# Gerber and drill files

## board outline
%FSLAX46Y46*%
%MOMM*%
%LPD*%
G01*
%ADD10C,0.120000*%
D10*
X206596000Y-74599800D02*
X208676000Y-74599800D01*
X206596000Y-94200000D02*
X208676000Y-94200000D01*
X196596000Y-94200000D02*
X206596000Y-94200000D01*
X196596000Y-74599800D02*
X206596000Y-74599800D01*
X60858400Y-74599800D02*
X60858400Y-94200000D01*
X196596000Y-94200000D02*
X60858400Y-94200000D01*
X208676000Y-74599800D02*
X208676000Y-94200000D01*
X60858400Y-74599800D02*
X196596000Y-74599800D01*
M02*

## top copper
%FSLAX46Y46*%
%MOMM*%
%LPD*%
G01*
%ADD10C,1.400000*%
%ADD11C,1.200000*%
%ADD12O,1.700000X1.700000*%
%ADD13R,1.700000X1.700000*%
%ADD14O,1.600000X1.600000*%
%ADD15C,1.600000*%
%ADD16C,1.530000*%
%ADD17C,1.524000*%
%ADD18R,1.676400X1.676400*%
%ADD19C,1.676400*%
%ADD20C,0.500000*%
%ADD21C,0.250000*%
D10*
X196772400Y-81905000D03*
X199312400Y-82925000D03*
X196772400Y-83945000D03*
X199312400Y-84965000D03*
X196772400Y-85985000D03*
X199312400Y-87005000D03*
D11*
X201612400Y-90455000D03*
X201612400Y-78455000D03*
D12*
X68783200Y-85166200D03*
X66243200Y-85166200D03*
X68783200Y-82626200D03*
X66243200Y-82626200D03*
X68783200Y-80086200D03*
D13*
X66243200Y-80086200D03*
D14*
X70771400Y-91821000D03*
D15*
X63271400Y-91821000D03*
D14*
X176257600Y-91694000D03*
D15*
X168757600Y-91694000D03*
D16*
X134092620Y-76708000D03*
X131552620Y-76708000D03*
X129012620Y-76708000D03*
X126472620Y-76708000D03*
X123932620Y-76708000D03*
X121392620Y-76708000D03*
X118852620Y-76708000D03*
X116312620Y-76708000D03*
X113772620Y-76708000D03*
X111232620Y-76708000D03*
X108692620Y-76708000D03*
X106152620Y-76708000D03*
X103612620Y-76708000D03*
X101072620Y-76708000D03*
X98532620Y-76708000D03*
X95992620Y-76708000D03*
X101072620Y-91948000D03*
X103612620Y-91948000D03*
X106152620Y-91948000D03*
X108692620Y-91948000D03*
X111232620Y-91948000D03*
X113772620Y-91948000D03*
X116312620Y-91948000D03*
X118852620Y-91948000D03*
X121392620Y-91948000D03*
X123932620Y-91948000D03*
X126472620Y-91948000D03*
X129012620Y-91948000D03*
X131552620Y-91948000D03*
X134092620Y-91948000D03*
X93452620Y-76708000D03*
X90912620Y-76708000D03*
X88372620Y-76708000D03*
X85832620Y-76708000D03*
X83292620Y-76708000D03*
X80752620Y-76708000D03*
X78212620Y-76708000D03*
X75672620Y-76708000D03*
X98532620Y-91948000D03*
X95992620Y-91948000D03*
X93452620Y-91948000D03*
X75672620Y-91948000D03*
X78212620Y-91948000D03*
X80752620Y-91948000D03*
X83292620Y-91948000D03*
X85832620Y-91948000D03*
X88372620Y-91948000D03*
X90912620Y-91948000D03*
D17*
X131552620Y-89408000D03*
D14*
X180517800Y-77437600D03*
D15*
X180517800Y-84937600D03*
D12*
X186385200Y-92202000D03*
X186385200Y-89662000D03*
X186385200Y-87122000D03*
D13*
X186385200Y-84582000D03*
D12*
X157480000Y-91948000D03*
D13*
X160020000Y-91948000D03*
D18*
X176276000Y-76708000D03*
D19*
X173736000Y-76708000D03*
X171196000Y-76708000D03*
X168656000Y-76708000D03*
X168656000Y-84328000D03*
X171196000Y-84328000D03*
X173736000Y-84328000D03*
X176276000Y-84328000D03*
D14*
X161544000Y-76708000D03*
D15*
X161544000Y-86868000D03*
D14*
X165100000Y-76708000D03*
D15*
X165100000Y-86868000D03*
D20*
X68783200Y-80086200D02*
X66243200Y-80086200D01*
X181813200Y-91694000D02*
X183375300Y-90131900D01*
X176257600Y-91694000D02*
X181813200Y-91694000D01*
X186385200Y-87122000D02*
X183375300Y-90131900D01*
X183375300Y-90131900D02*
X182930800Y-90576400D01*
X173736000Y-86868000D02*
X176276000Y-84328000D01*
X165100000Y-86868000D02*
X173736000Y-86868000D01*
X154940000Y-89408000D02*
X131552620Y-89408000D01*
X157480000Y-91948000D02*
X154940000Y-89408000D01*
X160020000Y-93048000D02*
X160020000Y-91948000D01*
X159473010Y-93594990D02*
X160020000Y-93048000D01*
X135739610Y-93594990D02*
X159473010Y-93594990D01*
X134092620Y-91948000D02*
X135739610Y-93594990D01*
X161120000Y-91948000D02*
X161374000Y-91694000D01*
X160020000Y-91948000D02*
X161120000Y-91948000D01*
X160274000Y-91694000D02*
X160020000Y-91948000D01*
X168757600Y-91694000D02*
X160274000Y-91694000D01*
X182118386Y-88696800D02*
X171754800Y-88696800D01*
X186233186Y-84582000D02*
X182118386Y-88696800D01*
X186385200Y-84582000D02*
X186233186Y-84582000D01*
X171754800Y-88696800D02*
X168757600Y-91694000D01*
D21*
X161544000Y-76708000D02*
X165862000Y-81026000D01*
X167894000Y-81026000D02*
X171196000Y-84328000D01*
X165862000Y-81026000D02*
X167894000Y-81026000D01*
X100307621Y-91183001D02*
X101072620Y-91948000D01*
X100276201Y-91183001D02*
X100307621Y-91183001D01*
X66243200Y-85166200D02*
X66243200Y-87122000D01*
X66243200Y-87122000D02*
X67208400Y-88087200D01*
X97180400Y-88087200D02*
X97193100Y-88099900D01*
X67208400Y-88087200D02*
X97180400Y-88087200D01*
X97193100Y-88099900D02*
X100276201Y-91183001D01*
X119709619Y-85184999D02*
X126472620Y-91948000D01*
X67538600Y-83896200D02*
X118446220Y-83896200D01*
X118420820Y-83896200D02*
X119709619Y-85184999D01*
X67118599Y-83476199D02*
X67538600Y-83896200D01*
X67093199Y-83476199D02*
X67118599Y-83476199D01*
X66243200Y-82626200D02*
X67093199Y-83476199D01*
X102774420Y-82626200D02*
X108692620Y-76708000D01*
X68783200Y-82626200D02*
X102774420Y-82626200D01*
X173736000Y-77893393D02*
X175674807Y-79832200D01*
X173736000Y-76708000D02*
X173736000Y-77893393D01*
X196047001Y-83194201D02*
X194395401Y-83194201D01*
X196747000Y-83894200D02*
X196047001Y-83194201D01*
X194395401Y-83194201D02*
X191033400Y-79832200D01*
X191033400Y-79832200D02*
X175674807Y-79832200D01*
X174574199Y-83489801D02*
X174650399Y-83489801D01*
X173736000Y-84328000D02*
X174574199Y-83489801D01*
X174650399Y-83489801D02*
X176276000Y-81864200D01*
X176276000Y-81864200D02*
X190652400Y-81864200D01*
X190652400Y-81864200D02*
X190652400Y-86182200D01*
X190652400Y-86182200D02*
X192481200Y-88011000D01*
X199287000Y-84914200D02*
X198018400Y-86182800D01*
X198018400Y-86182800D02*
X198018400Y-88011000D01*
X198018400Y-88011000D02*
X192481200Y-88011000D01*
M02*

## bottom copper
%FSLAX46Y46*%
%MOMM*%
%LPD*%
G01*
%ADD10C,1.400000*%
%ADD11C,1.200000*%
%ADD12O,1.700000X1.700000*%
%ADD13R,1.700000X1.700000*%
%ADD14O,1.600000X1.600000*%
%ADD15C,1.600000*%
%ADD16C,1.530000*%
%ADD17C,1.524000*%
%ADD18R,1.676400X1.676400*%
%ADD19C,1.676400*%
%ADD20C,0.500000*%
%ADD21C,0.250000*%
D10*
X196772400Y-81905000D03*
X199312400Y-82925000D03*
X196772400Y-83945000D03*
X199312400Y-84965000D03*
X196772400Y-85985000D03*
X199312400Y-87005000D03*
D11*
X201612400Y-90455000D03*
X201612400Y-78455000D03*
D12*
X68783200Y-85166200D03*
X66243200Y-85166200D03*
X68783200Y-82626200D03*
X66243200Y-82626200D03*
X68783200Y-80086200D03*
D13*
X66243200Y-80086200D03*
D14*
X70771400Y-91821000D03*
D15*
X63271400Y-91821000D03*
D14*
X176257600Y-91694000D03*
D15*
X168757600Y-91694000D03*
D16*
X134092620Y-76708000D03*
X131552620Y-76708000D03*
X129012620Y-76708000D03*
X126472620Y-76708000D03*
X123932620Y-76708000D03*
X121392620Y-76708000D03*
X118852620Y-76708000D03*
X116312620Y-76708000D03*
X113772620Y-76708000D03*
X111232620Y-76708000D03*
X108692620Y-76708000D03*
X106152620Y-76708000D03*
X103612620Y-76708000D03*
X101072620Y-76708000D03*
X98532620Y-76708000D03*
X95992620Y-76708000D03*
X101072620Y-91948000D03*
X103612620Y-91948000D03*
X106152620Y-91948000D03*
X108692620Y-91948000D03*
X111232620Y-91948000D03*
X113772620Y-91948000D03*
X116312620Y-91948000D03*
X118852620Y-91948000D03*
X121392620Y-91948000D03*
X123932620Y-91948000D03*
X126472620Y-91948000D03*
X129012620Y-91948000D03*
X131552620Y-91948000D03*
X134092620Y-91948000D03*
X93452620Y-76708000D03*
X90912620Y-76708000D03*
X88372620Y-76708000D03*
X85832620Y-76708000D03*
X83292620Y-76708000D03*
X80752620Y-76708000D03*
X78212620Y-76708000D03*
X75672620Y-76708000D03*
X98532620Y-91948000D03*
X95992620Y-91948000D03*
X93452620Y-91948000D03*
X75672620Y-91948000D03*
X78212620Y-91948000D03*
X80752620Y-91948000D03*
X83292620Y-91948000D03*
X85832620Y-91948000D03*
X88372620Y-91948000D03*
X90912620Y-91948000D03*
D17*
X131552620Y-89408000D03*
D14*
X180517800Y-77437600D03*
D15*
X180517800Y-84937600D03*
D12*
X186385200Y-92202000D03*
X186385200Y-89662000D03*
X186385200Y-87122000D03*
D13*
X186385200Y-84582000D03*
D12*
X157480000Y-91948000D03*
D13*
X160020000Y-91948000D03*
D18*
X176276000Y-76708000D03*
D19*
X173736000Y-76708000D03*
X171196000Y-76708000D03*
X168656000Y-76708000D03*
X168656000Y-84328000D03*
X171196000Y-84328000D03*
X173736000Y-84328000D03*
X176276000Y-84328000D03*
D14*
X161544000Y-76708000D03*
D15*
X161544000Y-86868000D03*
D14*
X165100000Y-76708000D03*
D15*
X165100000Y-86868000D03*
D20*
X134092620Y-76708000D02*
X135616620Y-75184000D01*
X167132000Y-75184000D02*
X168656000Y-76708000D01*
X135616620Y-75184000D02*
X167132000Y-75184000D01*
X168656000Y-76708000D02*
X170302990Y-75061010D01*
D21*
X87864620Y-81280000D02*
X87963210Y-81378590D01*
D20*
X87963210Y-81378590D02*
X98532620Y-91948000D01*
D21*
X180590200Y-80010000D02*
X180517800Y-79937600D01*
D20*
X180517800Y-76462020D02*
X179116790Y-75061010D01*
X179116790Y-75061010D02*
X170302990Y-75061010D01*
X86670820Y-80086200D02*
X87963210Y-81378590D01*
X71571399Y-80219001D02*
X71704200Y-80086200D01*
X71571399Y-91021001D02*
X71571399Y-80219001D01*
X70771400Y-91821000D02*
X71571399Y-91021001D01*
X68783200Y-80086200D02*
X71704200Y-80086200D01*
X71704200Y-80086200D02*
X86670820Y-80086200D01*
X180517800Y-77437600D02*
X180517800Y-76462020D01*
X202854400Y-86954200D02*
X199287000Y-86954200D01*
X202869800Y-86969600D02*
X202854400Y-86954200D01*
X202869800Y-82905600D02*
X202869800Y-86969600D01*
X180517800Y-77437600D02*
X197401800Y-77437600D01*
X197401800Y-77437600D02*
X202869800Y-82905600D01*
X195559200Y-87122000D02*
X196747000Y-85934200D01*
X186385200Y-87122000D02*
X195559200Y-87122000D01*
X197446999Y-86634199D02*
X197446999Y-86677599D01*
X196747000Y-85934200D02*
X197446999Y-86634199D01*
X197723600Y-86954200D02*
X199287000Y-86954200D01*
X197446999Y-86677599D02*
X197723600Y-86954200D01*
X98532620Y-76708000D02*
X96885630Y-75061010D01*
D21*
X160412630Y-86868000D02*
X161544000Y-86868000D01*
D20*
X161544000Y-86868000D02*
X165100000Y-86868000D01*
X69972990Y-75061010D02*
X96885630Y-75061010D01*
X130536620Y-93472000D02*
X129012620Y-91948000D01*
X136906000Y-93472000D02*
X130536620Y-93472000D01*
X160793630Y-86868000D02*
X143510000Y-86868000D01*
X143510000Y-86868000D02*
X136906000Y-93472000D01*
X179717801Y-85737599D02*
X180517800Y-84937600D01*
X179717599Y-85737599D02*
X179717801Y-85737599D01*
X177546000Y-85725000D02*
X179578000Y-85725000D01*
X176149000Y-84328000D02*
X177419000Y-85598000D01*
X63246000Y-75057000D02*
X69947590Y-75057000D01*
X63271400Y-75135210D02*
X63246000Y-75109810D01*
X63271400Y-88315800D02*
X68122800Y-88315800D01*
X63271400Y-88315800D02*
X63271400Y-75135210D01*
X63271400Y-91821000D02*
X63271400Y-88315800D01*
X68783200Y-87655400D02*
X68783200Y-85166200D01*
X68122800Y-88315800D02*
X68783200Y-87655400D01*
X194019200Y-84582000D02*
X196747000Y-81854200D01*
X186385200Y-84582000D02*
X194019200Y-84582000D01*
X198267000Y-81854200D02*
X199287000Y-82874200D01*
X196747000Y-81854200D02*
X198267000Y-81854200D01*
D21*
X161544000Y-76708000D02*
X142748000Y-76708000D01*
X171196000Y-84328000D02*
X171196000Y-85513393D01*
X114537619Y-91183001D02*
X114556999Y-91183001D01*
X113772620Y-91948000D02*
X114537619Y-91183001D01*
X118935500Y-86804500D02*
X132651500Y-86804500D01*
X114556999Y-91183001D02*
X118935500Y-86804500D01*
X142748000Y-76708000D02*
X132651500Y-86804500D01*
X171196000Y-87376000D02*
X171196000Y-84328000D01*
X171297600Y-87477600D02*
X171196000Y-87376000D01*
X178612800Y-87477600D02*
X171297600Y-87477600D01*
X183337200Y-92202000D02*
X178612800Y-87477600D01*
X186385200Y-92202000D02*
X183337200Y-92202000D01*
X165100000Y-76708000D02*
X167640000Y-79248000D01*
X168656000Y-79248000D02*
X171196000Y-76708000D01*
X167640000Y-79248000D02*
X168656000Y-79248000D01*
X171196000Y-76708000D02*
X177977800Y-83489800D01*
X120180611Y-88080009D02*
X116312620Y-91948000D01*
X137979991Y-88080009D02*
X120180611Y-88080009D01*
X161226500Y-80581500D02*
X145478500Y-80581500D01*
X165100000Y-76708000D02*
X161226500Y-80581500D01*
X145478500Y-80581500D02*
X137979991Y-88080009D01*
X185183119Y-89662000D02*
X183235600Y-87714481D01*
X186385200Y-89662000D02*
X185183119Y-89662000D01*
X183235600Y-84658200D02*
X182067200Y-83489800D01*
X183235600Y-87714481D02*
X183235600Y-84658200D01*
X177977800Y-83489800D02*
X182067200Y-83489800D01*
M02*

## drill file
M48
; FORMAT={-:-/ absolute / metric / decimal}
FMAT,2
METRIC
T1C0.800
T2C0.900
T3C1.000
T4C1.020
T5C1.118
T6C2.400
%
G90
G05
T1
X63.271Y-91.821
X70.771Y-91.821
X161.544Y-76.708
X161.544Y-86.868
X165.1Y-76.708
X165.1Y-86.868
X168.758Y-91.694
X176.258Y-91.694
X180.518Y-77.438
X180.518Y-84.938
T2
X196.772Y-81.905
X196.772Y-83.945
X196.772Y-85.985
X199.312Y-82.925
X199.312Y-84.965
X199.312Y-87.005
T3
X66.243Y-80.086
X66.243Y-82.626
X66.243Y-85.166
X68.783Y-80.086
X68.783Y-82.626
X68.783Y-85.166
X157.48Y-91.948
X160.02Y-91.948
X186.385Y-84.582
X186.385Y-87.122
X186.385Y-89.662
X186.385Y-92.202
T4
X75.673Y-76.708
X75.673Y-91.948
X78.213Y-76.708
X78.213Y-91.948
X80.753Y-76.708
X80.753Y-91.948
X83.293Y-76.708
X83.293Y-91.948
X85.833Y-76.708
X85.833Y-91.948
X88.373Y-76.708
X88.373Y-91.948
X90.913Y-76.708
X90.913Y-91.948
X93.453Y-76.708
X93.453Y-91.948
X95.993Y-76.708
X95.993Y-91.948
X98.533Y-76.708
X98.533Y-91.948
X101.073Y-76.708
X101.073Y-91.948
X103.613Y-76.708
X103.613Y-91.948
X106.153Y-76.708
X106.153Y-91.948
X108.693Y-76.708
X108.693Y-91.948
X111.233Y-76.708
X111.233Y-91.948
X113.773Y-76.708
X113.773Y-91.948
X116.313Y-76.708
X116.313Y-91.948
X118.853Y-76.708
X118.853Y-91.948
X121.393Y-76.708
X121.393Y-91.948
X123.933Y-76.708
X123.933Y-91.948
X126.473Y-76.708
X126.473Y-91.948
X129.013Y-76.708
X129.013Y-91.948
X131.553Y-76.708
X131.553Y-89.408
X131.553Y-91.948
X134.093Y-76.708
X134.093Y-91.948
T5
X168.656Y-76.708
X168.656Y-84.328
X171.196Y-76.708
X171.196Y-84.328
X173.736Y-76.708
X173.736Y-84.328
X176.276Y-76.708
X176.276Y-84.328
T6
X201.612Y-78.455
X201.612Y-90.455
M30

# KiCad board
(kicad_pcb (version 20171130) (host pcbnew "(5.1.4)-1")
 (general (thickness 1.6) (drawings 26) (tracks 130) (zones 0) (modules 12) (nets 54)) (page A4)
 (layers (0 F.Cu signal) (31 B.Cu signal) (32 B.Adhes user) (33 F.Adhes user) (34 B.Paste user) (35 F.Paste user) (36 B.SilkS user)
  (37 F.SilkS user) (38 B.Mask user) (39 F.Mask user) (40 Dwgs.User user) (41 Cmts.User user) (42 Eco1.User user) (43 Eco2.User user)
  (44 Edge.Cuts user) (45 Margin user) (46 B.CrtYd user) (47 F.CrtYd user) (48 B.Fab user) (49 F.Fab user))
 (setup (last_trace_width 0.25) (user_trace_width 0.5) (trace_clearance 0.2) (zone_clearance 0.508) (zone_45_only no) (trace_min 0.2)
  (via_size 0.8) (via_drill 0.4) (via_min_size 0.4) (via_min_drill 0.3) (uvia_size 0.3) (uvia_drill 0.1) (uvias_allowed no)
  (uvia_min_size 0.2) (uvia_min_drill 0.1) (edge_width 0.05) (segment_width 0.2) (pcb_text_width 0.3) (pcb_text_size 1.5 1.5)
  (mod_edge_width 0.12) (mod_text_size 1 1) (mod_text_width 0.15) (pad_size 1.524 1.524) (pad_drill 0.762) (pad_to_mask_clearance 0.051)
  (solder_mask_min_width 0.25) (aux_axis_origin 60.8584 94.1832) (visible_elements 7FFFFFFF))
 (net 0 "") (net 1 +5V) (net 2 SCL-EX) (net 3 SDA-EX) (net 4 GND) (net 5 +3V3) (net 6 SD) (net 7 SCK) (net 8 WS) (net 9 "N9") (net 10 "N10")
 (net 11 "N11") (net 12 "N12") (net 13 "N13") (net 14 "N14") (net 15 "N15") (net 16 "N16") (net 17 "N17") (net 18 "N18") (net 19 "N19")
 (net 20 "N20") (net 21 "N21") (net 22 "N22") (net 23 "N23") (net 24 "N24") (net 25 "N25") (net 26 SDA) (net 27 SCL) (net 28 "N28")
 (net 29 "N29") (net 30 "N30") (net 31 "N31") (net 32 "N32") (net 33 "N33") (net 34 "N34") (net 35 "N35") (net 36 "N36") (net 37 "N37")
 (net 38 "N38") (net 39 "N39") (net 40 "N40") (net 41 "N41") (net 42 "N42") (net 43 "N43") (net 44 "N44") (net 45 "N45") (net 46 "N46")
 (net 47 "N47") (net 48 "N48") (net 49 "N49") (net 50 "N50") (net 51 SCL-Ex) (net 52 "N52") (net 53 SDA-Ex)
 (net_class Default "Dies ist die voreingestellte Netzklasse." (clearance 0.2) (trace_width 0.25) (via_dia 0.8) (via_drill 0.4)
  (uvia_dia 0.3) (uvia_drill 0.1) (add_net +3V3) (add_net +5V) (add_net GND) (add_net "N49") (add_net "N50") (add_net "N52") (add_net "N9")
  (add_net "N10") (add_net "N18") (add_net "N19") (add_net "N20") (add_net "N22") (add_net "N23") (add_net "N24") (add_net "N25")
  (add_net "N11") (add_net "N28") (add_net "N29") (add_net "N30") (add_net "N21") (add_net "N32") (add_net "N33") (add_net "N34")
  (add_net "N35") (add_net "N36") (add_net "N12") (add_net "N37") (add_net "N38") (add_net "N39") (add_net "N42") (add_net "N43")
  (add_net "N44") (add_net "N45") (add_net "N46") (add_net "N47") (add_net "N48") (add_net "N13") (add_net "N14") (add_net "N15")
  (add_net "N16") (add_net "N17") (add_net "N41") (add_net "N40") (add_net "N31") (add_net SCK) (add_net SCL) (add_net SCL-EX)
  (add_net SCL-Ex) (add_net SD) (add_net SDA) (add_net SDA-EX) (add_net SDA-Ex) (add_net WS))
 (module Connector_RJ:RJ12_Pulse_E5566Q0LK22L (layer F.Cu) (at 200.8124 84.455 90)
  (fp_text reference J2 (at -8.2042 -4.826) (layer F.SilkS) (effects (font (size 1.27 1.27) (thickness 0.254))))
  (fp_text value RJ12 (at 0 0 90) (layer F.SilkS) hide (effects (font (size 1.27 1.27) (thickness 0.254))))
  (pad 1 thru_hole circle (at 2.55 -4.04 180) (size 1.4 1.4) (drill 0.9) (layers *.Cu *.Mask F.SilkS) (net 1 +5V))
  (pad 2 thru_hole circle (at 1.53 -1.5 180) (size 1.4 1.4) (drill 0.9) (layers *.Cu *.Mask F.SilkS) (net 1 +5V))
  (pad 3 thru_hole circle (at 0.51 -4.04 180) (size 1.4 1.4) (drill 0.9) (layers *.Cu *.Mask F.SilkS) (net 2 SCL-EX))
  (pad 4 thru_hole circle (at -0.51 -1.5 180) (size 1.4 1.4) (drill 0.9) (layers *.Cu *.Mask F.SilkS) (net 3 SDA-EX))
  (pad 5 thru_hole circle (at -1.53 -4.04 180) (size 1.4 1.4) (drill 0.9) (layers *.Cu *.Mask F.SilkS) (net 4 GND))
  (pad 6 thru_hole circle (at -2.55 -1.5 180) (size 1.4 1.4) (drill 0.9) (layers *.Cu *.Mask F.SilkS) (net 4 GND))
  (pad 7 thru_hole circle (at -6 0.8 180) (size 1.2 1.2) (drill 2.4) (layers *.Cu *.Mask F.SilkS))
  (pad 8 thru_hole circle (at 6 0.8 180) (size 1.2 1.2) (drill 2.4) (layers *.Cu *.Mask F.SilkS)))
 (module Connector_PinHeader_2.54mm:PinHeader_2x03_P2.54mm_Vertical (layer F.Cu) (at 66.2432 80.0862)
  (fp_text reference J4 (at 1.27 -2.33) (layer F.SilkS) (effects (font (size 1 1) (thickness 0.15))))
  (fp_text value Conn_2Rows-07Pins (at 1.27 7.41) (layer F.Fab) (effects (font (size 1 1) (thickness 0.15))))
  (pad 6 thru_hole oval (at 2.54 5.08) (size 1.7 1.7) (drill 1) (layers *.Cu *.Mask) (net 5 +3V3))
  (pad 5 thru_hole oval (at 0 5.08) (size 1.7 1.7) (drill 1) (layers *.Cu *.Mask) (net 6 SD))
  (pad 4 thru_hole oval (at 2.54 2.54) (size 1.7 1.7) (drill 1) (layers *.Cu *.Mask) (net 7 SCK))
  (pad 3 thru_hole oval (at 0 2.54) (size 1.7 1.7) (drill 1) (layers *.Cu *.Mask) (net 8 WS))
  (pad 2 thru_hole oval (at 2.54 0) (size 1.7 1.7) (drill 1) (layers *.Cu *.Mask) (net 4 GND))
  (pad 1 thru_hole rect (at 0 0) (size 1.7 1.7) (drill 1) (layers *.Cu *.Mask) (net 4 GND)))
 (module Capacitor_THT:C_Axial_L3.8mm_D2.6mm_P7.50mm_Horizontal (layer F.Cu) (at 63.2714 91.821)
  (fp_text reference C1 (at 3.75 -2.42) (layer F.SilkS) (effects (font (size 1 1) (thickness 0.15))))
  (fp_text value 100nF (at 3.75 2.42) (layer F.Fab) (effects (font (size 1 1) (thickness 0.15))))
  (pad 2 thru_hole oval (at 7.5 0) (size 1.6 1.6) (drill 0.8) (layers *.Cu *.Mask) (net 4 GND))
  (pad 1 thru_hole circle (at 0 0) (size 1.6 1.6) (drill 0.8) (layers *.Cu *.Mask) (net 5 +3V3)))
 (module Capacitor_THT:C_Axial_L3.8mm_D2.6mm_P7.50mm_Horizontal (layer F.Cu) (at 168.7576 91.694)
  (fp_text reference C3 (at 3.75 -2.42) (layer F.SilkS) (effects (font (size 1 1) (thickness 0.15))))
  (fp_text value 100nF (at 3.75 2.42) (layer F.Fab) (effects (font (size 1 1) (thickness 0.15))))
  (pad 2 thru_hole oval (at 7.5 0) (size 1.6 1.6) (drill 0.8) (layers *.Cu *.Mask) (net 4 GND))
  (pad 1 thru_hole circle (at 0 0) (size 1.6 1.6) (drill 0.8) (layers *.Cu *.Mask) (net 1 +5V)))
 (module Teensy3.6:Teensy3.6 (layer F.Cu) (at 104.88262 84.328 270)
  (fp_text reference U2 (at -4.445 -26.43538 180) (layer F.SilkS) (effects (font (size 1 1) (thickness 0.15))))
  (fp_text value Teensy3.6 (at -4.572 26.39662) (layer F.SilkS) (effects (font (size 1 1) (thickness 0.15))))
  (pad GND_1 thru_hole circle (at -7.62 -29.21 270) (size 1.53 1.53) (drill 1.02) (layers *.Cu *.Mask) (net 4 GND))
  (pad 0 thru_hole circle (at -7.62 -26.67 270) (size 1.53 1.53) (drill 1.02) (layers *.Cu *.Mask) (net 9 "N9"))
  (pad 1 thru_hole circle (at -7.62 -24.13 270) (size 1.53 1.53) (drill 1.02) (layers *.Cu *.Mask) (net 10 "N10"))
  (pad 2 thru_hole circle (at -7.62 -21.59 270) (size 1.53 1.53) (drill 1.02) (layers *.Cu *.Mask) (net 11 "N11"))
  (pad 3 thru_hole circle (at -7.62 -19.05 270) (size 1.53 1.53) (drill 1.02) (layers *.Cu *.Mask) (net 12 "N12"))
  (pad 4 thru_hole circle (at -7.62 -16.51 270) (size 1.53 1.53) (drill 1.02) (layers *.Cu *.Mask) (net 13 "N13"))
  (pad 5 thru_hole circle (at -7.62 -13.97 270) (size 1.53 1.53) (drill 1.02) (layers *.Cu *.Mask) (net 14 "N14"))
  (pad 6 thru_hole circle (at -7.62 -11.43 270) (size 1.53 1.53) (drill 1.02) (layers *.Cu *.Mask) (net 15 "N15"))
  (pad 7 thru_hole circle (at -7.62 -8.89 270) (size 1.53 1.53) (drill 1.02) (layers *.Cu *.Mask) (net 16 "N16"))
  (pad 8 thru_hole circle (at -7.62 -6.35 270) (size 1.53 1.53) (drill 1.02) (layers *.Cu *.Mask) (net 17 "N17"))
  (pad 9 thru_hole circle (at -7.62 -3.81 270) (size 1.53 1.53) (drill 1.02) (layers *.Cu *.Mask) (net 7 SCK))
  (pad 10 thru_hole circle (at -7.62 -1.27 270) (size 1.53 1.53) (drill 1.02) (layers *.Cu *.Mask) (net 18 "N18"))
  (pad 11 thru_hole circle (at -7.62 1.27 270) (size 1.53 1.53) (drill 1.02) (layers *.Cu *.Mask) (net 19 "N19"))
  (pad 12 thru_hole circle (at -7.62 3.81 270) (size 1.53 1.53) (drill 1.02) (layers *.Cu *.Mask) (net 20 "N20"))
  (pad 3V3_1 thru_hole circle (at -7.62 6.35 270) (size 1.53 1.53) (drill 1.02) (layers *.Cu *.Mask) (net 5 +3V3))
  (pad 24 thru_hole circle (at -7.62 8.89 270) (size 1.53 1.53) (drill 1.02) (layers *.Cu *.Mask) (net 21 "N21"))
  (pad 13 thru_hole circle (at 7.62 3.81 270) (size 1.53 1.53) (drill 1.02) (layers *.Cu *.Mask) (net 6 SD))
  (pad 14 thru_hole circle (at 7.62 1.27 270) (size 1.53 1.53) (drill 1.02) (layers *.Cu *.Mask) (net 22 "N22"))
  (pad 15 thru_hole circle (at 7.62 -1.27 270) (size 1.53 1.53) (drill 1.02) (layers *.Cu *.Mask) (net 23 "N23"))
  (pad 16 thru_hole circle (at 7.62 -3.81 270) (size 1.53 1.53) (drill 1.02) (layers *.Cu *.Mask) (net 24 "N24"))
  (pad 17 thru_hole circle (at 7.62 -6.35 270) (size 1.53 1.53) (drill 1.02) (layers *.Cu *.Mask) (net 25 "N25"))
  (pad 18 thru_hole circle (at 7.62 -8.89 270) (size 1.53 1.53) (drill 1.02) (layers *.Cu *.Mask) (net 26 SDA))
  (pad 19 thru_hole circle (at 7.62 -11.43 270) (size 1.53 1.53) (drill 1.02) (layers *.Cu *.Mask) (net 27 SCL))
  (pad 20 thru_hole circle (at 7.62 -13.97 270) (size 1.53 1.53) (drill 1.02) (layers *.Cu *.Mask) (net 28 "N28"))
  (pad 21 thru_hole circle (at 7.62 -16.51 270) (size 1.53 1.53) (drill 1.02) (layers *.Cu *.Mask) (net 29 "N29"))
  (pad 22 thru_hole circle (at 7.62 -19.05 270) (size 1.53 1.53) (drill 1.02) (layers *.Cu *.Mask) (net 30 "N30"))
  (pad 23 thru_hole circle (at 7.62 -21.59 270) (size 1.53 1.53) (drill 1.02) (layers *.Cu *.Mask) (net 8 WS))
  (pad 3V3_2 thru_hole circle (at 7.62 -24.13 270) (size 1.53 1.53) (drill 1.02) (layers *.Cu *.Mask) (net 5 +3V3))
  (pad AGND thru_hole circle (at 7.62 -26.67 270) (size 1.53 1.53) (drill 1.02) (layers *.Cu *.Mask) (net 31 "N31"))
  (pad VIN thru_hole circle (at 7.62 -29.21 270) (size 1.53 1.53) (drill 1.02) (layers *.Cu *.Mask) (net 1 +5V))
  (pad 25 thru_hole circle (at -7.62 11.43 270) (size 1.53 1.53) (drill 1.02) (layers *.Cu *.Mask) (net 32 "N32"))
  (pad 26 thru_hole circle (at -7.62 13.97 270) (size 1.53 1.53) (drill 1.02) (layers *.Cu *.Mask) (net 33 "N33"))
  (pad 27 thru_hole circle (at -7.62 16.51 270) (size 1.53 1.53) (drill 1.02) (layers *.Cu *.Mask) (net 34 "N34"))
  (pad 28 thru_hole circle (at -7.62 19.05 270) (size 1.53 1.53) (drill 1.02) (layers *.Cu *.Mask) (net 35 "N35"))
  (pad 29 thru_hole circle (at -7.62 21.59 270) (size 1.53 1.53) (drill 1.02) (layers *.Cu *.Mask) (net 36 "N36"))
  (pad 30 thru_hole circle (at -7.62 24.13 270) (size 1.53 1.53) (drill 1.02) (layers *.Cu *.Mask) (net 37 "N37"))
  (pad 31 thru_hole circle (at -7.62 26.67 270) (size 1.53 1.53) (drill 1.02) (layers *.Cu *.Mask) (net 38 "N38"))
  (pad 32 thru_hole circle (at -7.62 29.21 270) (size 1.53 1.53) (drill 1.02) (layers *.Cu *.Mask) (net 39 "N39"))
  (pad GND_2 thru_hole circle (at 7.62 6.35 270) (size 1.53 1.53) (drill 1.02) (layers *.Cu *.Mask) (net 4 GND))
  (pad A22 thru_hole circle (at 7.62 8.89 270) (size 1.53 1.53) (drill 1.02) (layers *.Cu *.Mask) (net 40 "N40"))
  (pad A21 thru_hole circle (at 7.62 11.43 270) (size 1.53 1.53) (drill 1.02) (layers *.Cu *.Mask) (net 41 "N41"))
  (pad 33 thru_hole circle (at 7.62 29.21 270) (size 1.53 1.53) (drill 1.02) (layers *.Cu *.Mask) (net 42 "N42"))
  (pad 34 thru_hole circle (at 7.62 26.67 270) (size 1.53 1.53) (drill 1.02) (layers *.Cu *.Mask) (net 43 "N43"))
  (pad 35 thru_hole circle (at 7.62 24.13 270) (size 1.53 1.53) (drill 1.02) (layers *.Cu *.Mask) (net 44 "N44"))
  (pad 36 thru_hole circle (at 7.62 21.59 270) (size 1.53 1.53) (drill 1.02) (layers *.Cu *.Mask) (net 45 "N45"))
  (pad 37 thru_hole circle (at 7.62 19.05 270) (size 1.53 1.53) (drill 1.02) (layers *.Cu *.Mask) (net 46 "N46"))
  (pad 38 thru_hole circle (at 7.62 16.51 270) (size 1.53 1.53) (drill 1.02) (layers *.Cu *.Mask) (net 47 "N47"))
  (pad 39 thru_hole circle (at 7.62 13.97 270) (size 1.53 1.53) (drill 1.02) (layers *.Cu *.Mask) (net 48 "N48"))
  (pad VUSB thru_hole circle (at 5.08 -26.67 270) (size 1.524 1.524) (drill 1.02) (layers *.Cu *.Mask) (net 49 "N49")))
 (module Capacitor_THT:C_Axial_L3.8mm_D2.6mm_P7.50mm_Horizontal (layer F.Cu) (at 180.5178 84.9376 90)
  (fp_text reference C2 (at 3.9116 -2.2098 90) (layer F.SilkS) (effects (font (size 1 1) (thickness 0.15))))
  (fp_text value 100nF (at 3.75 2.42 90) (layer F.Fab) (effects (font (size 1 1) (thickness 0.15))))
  (pad 2 thru_hole oval (at 7.5 0 90) (size 1.6 1.6) (drill 0.8) (layers *.Cu *.Mask) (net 4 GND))
  (pad 1 thru_hole circle (at 0 0 90) (size 1.6 1.6) (drill 0.8) (layers *.Cu *.Mask) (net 5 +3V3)))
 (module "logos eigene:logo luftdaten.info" (layer F.Cu) (at 143.1798 88.5698)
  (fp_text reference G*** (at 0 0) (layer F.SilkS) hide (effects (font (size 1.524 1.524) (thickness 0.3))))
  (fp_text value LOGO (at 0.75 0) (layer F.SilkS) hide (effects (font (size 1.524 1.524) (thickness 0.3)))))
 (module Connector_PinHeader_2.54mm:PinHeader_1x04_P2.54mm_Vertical (layer F.Cu) (at 186.3852 84.582)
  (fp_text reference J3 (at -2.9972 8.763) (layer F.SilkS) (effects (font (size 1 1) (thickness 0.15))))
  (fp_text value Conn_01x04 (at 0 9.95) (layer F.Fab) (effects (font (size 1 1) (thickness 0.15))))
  (pad 4 thru_hole oval (at 0 7.62) (size 1.7 1.7) (drill 1) (layers *.Cu *.Mask) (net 26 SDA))
  (pad 3 thru_hole oval (at 0 5.08) (size 1.7 1.7) (drill 1) (layers *.Cu *.Mask) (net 27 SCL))
  (pad 2 thru_hole oval (at 0 2.54) (size 1.7 1.7) (drill 1) (layers *.Cu *.Mask) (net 4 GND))
  (pad 1 thru_hole rect (at 0 0) (size 1.7 1.7) (drill 1) (layers *.Cu *.Mask) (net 1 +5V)))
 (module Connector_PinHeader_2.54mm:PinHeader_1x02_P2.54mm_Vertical (layer F.Cu) (at 160.02 91.948 270)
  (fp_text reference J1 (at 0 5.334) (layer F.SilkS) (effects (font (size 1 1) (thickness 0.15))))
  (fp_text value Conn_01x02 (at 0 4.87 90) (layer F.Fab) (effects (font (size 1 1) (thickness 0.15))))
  (pad 2 thru_hole oval (at 0 2.54 270) (size 1.7 1.7) (drill 1) (layers *.Cu *.Mask) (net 49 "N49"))
  (pad 1 thru_hole rect (at 0 0 270) (size 1.7 1.7) (drill 1) (layers *.Cu *.Mask) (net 1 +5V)))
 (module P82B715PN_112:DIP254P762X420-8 (layer F.Cu) (at 168.656 84.328 270)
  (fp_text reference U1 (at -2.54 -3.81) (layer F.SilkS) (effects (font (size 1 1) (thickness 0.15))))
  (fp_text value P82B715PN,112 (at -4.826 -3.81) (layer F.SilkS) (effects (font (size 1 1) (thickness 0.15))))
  (pad 1 thru_hole rect (at -7.62 -7.62 270) (size 1.6764 1.6764) (drill 1.1176) (layers *.Cu *.Mask) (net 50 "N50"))
  (pad 2 thru_hole circle (at -7.62 -5.08 270) (size 1.6764 1.6764) (drill 1.1176) (layers *.Cu *.Mask) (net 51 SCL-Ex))
  (pad 3 thru_hole circle (at -7.62 -2.54 270) (size 1.6764 1.6764) (drill 1.1176) (layers *.Cu *.Mask) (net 27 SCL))
  (pad 4 thru_hole circle (at -7.62 0 270) (size 1.6764 1.6764) (drill 1.1176) (layers *.Cu *.Mask) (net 4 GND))
  (pad 5 thru_hole circle (at 0 0 270) (size 1.6764 1.6764) (drill 1.1176) (layers *.Cu *.Mask) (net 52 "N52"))
  (pad 6 thru_hole circle (at 0 -2.54 270) (size 1.6764 1.6764) (drill 1.1176) (layers *.Cu *.Mask) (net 26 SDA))
  (pad 7 thru_hole circle (at 0 -5.08 270) (size 1.6764 1.6764) (drill 1.1176) (layers *.Cu *.Mask) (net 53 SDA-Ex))
  (pad 8 thru_hole circle (at 0 -7.62 270) (size 1.6764 1.6764) (drill 1.1176) (layers *.Cu *.Mask) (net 5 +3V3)))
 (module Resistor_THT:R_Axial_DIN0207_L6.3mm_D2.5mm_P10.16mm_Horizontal (layer F.Cu) (at 161.544 86.868 90)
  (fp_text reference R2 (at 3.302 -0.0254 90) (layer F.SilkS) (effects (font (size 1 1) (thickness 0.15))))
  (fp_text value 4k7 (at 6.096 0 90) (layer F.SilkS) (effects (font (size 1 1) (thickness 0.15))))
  (pad 2 thru_hole oval (at 10.16 0 90) (size 1.6 1.6) (drill 0.8) (layers *.Cu *.Mask) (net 26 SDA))
  (pad 1 thru_hole circle (at 0 0 90) (size 1.6 1.6) (drill 0.8) (layers *.Cu *.Mask) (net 5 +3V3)))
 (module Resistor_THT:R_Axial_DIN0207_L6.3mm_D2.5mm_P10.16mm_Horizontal (layer F.Cu) (at 165.1 86.868 90)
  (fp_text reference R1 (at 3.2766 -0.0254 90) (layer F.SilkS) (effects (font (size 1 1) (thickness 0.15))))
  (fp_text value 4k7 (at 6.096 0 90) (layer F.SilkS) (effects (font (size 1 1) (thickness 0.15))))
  (pad 2 thru_hole oval (at 10.16 0 90) (size 1.6 1.6) (drill 0.8) (layers *.Cu *.Mask) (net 27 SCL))
  (pad 1 thru_hole circle (at 0 0 90) (size 1.6 1.6) (drill 0.8) (layers *.Cu *.Mask) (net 5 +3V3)))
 (gr_line (start 206.596 74.5998) (end 208.676 74.5998) (layer Edge.Cuts) (width 0.12))
 (gr_line (start 206.596 94.2) (end 208.676 94.2) (layer Edge.Cuts) (width 0.12))
 (gr_line (start 196.596 94.2) (end 206.596 94.2) (layer Edge.Cuts) (width 0.12))
 (gr_line (start 196.596 74.5998) (end 206.596 74.5998) (layer Edge.Cuts) (width 0.12))
 (gr_line (start 60.8584 74.5998) (end 60.8584 94.2) (layer Edge.Cuts) (width 0.12))
 (gr_line (start 196.596 94.2) (end 60.8584 94.2) (layer Edge.Cuts) (width 0.12))
 (gr_line (start 208.676 74.5998) (end 208.676 94.2) (layer Edge.Cuts) (width 0.12))
 (gr_line (start 60.8584 74.5998) (end 196.596 74.5998) (layer Edge.Cuts) (width 0.12))
 (segment (start 134.09262 76.708) (end 135.61662 75.184) (width 0.5) (layer B.Cu) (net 4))
 (segment (start 167.132 75.184) (end 168.656 76.708) (width 0.5) (layer B.Cu) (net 4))
 (segment (start 135.61662 75.184) (end 167.132 75.184) (width 0.5) (layer B.Cu) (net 4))
 (segment (start 168.656 76.708) (end 170.30299 75.06101) (width 0.5) (layer B.Cu) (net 4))
 (segment (start 87.86462 81.28) (end 87.96321 81.37859) (width 0.25) (layer B.Cu) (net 4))
 (segment (start 87.96321 81.37859) (end 98.53262 91.948) (width 0.5) (layer B.Cu) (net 4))
 (segment (start 180.5902 80.01) (end 180.5178 79.9376) (width 0.25) (layer B.Cu) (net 4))
 (segment (start 180.5178 76.46202) (end 179.11679 75.06101) (width 0.5) (layer B.Cu) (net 4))
 (segment (start 179.11679 75.06101) (end 170.30299 75.06101) (width 0.5) (layer B.Cu) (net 4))
 (segment (start 86.67082 80.0862) (end 87.96321 81.37859) (width 0.5) (layer B.Cu) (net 4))
 (segment (start 68.7832 80.0862) (end 66.2432 80.0862) (width 0.5) (layer F.Cu) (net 4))
 (segment (start 71.571399 80.219001) (end 71.7042 80.0862) (width 0.5) (layer B.Cu) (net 4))
 (segment (start 71.571399 91.021001) (end 71.571399 80.219001) (width 0.5) (layer B.Cu) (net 4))
 (segment (start 70.7714 91.821) (end 71.571399 91.021001) (width 0.5) (layer B.Cu) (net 4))
 (segment (start 68.7832 80.0862) (end 71.7042 80.0862) (width 0.5) (layer B.Cu) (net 4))
 (segment (start 71.7042 80.0862) (end 86.67082 80.0862) (width 0.5) (layer B.Cu) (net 4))
 (segment (start 181.8132 91.694) (end 183.3753 90.1319) (width 0.5) (layer F.Cu) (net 4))
 (segment (start 176.2576 91.694) (end 181.8132 91.694) (width 0.5) (layer F.Cu) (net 4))
 (segment (start 186.3852 87.122) (end 183.3753 90.1319) (width 0.5) (layer F.Cu) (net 4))
 (segment (start 183.3753 90.1319) (end 182.9308 90.5764) (width 0.5) (layer F.Cu) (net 4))
 (segment (start 180.5178 77.4376) (end 180.5178 76.46202) (width 0.5) (layer B.Cu) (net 4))
 (segment (start 202.8544 86.9542) (end 199.287 86.9542) (width 0.5) (layer B.Cu) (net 4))
 (segment (start 202.8698 86.9696) (end 202.8544 86.9542) (width 0.5) (layer B.Cu) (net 4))
 (segment (start 202.8698 82.9056) (end 202.8698 86.9696) (width 0.5) (layer B.Cu) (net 4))
 (segment (start 180.5178 77.4376) (end 197.4018 77.4376) (width 0.5) (layer B.Cu) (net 4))
 (segment (start 197.4018 77.4376) (end 202.8698 82.9056) (width 0.5) (layer B.Cu) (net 4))
 (segment (start 195.5592 87.122) (end 196.747 85.9342) (width 0.5) (layer B.Cu) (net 4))
 (segment (start 186.3852 87.122) (end 195.5592 87.122) (width 0.5) (layer B.Cu) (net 4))
 (segment (start 197.446999 86.634199) (end 197.446999 86.677599) (width 0.5) (layer B.Cu) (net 4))
 (segment (start 196.747 85.9342) (end 197.446999 86.634199) (width 0.5) (layer B.Cu) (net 4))
 (segment (start 197.7236 86.9542) (end 199.287 86.9542) (width 0.5) (layer B.Cu) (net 4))
 (segment (start 197.446999 86.677599) (end 197.7236 86.9542) (width 0.5) (layer B.Cu) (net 4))
 (segment (start 98.53262 76.708) (end 96.88563 75.06101) (width 0.5) (layer B.Cu) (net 5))
 (segment (start 160.41263 86.868) (end 161.544 86.868) (width 0.25) (layer B.Cu) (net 5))
 (segment (start 161.544 86.868) (end 165.1 86.868) (width 0.5) (layer B.Cu) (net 5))
 (segment (start 173.736 86.868) (end 176.276 84.328) (width 0.5) (layer F.Cu) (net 5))
 (segment (start 165.1 86.868) (end 173.736 86.868) (width 0.5) (layer F.Cu) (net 5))
 (segment (start 69.97299 75.06101) (end 96.88563 75.06101) (width 0.5) (layer B.Cu) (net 5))
 (segment (start 130.53662 93.472) (end 129.01262 91.948) (width 0.5) (layer B.Cu) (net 5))
 (segment (start 136.906 93.472) (end 130.53662 93.472) (width 0.5) (layer B.Cu) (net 5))
 (segment (start 160.79363 86.868) (end 143.51 86.868) (width 0.5) (layer B.Cu) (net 5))
 (segment (start 143.51 86.868) (end 136.906 93.472) (width 0.5) (layer B.Cu) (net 5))
 (segment (start 179.717801 85.737599) (end 180.5178 84.9376) (width 0.5) (layer B.Cu) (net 5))
 (segment (start 179.717599 85.737599) (end 179.717801 85.737599) (width 0.5) (layer B.Cu) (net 5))
 (segment (start 177.546 85.725) (end 179.578 85.725) (width 0.5) (layer B.Cu) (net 5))
 (segment (start 176.149 84.328) (end 177.419 85.598) (width 0.5) (layer B.Cu) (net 5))
 (segment (start 63.246 75.057) (end 69.94759 75.057) (width 0.5) (layer B.Cu) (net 5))
 (segment (start 63.2714 75.13521) (end 63.246 75.10981) (width 0.5) (layer B.Cu) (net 5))
 (segment (start 63.2714 88.3158) (end 68.1228 88.3158) (width 0.5) (layer B.Cu) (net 5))
 (segment (start 63.2714 88.3158) (end 63.2714 75.13521) (width 0.5) (layer B.Cu) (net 5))
 (segment (start 63.2714 91.821) (end 63.2714 88.3158) (width 0.5) (layer B.Cu) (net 5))
 (segment (start 68.7832 87.6554) (end 68.7832 85.1662) (width 0.5) (layer B.Cu) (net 5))
 (segment (start 68.1228 88.3158) (end 68.7832 87.6554) (width 0.5) (layer B.Cu) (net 5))
 (segment (start 154.94 89.408) (end 131.55262 89.408) (width 0.5) (layer F.Cu) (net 49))
 (segment (start 157.48 91.948) (end 154.94 89.408) (width 0.5) (layer F.Cu) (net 49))
 (segment (start 160.02 93.048) (end 160.02 91.948) (width 0.5) (layer F.Cu) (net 1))
 (segment (start 159.47301 93.59499) (end 160.02 93.048) (width 0.5) (layer F.Cu) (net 1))
 (segment (start 135.73961 93.59499) (end 159.47301 93.59499) (width 0.5) (layer F.Cu) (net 1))
 (segment (start 134.09262 91.948) (end 135.73961 93.59499) (width 0.5) (layer F.Cu) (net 1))
 (segment (start 161.12 91.948) (end 161.374 91.694) (width 0.5) (layer F.Cu) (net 1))
 (segment (start 160.02 91.948) (end 161.12 91.948) (width 0.5) (layer F.Cu) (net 1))
 (segment (start 160.274 91.694) (end 160.02 91.948) (width 0.5) (layer F.Cu) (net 1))
 (segment (start 168.7576 91.694) (end 160.274 91.694) (width 0.5) (layer F.Cu) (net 1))
 (segment (start 182.118386 88.6968) (end 171.7548 88.6968) (width 0.5) (layer F.Cu) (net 1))
 (segment (start 186.233186 84.582) (end 182.118386 88.6968) (width 0.5) (layer F.Cu) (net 1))
 (segment (start 186.3852 84.582) (end 186.233186 84.582) (width 0.5) (layer F.Cu) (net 1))
 (segment (start 171.7548 88.6968) (end 168.7576 91.694) (width 0.5) (layer F.Cu) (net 1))
 (segment (start 194.0192 84.582) (end 196.747 81.8542) (width 0.5) (layer B.Cu) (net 1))
 (segment (start 186.3852 84.582) (end 194.0192 84.582) (width 0.5) (layer B.Cu) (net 1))
 (segment (start 198.267 81.8542) (end 199.287 82.8742) (width 0.5) (layer B.Cu) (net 1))
 (segment (start 196.747 81.8542) (end 198.267 81.8542) (width 0.5) (layer B.Cu) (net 1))
 (segment (start 161.544 76.708) (end 142.748 76.708) (width 0.25) (layer B.Cu) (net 26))
 (segment (start 161.544 76.708) (end 165.862 81.026) (width 0.25) (layer F.Cu) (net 26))
 (segment (start 167.894 81.026) (end 171.196 84.328) (width 0.25) (layer F.Cu) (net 26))
 (segment (start 165.862 81.026) (end 167.894 81.026) (width 0.25) (layer F.Cu) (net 26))
 (segment (start 171.196 84.328) (end 171.196 85.513393) (width 0.25) (layer B.Cu) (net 26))
 (segment (start 114.537619 91.183001) (end 114.556999 91.183001) (width 0.25) (layer B.Cu) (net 26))
 (segment (start 113.77262 91.948) (end 114.537619 91.183001) (width 0.25) (layer B.Cu) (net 26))
 (segment (start 118.9355 86.8045) (end 132.6515 86.8045) (width 0.25) (layer B.Cu) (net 26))
 (segment (start 114.556999 91.183001) (end 118.9355 86.8045) (width 0.25) (layer B.Cu) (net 26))
 (segment (start 142.748 76.708) (end 132.6515 86.8045) (width 0.25) (layer B.Cu) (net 26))
 (segment (start 171.196 87.376) (end 171.196 84.328) (width 0.25) (layer B.Cu) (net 26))
 (segment (start 171.2976 87.4776) (end 171.196 87.376) (width 0.25) (layer B.Cu) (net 26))
 (segment (start 178.6128 87.4776) (end 171.2976 87.4776) (width 0.25) (layer B.Cu) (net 26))
 (segment (start 183.3372 92.202) (end 178.6128 87.4776) (width 0.25) (layer B.Cu) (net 26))
 (segment (start 186.3852 92.202) (end 183.3372 92.202) (width 0.25) (layer B.Cu) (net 26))
 (segment (start 165.1 76.708) (end 167.64 79.248) (width 0.25) (layer B.Cu) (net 27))
 (segment (start 168.656 79.248) (end 171.196 76.708) (width 0.25) (layer B.Cu) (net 27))
 (segment (start 167.64 79.248) (end 168.656 79.248) (width 0.25) (layer B.Cu) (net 27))
 (segment (start 171.196 76.708) (end 177.9778 83.4898) (width 0.25) (layer B.Cu) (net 27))
 (segment (start 120.180611 88.080009) (end 116.31262 91.948) (width 0.25) (layer B.Cu) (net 27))
 (segment (start 137.979991 88.080009) (end 120.180611 88.080009) (width 0.25) (layer B.Cu) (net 27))
 (segment (start 161.2265 80.5815) (end 145.4785 80.5815) (width 0.25) (layer B.Cu) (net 27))
 (segment (start 165.1 76.708) (end 161.2265 80.5815) (width 0.25) (layer B.Cu) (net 27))
 (segment (start 145.4785 80.5815) (end 137.979991 88.080009) (width 0.25) (layer B.Cu) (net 27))
 (segment (start 185.183119 89.662) (end 183.2356 87.714481) (width 0.25) (layer B.Cu) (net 27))
 (segment (start 186.3852 89.662) (end 185.183119 89.662) (width 0.25) (layer B.Cu) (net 27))
 (segment (start 183.2356 84.6582) (end 182.0672 83.4898) (width 0.25) (layer B.Cu) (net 27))
 (segment (start 183.2356 87.714481) (end 183.2356 84.6582) (width 0.25) (layer B.Cu) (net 27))
 (segment (start 177.9778 83.4898) (end 182.0672 83.4898) (width 0.25) (layer B.Cu) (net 27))
 (segment (start 100.307621 91.183001) (end 101.07262 91.948) (width 0.25) (layer F.Cu) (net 6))
 (segment (start 100.276201 91.183001) (end 100.307621 91.183001) (width 0.25) (layer F.Cu) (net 6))
 (segment (start 66.2432 85.1662) (end 66.2432 87.122) (width 0.25) (layer F.Cu) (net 6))
 (segment (start 66.2432 87.122) (end 67.2084 88.0872) (width 0.25) (layer F.Cu) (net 6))
 (segment (start 97.1804 88.0872) (end 97.1931 88.0999) (width 0.25) (layer F.Cu) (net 6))
 (segment (start 67.2084 88.0872) (end 97.1804 88.0872) (width 0.25) (layer F.Cu) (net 6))
 (segment (start 97.1931 88.0999) (end 100.276201 91.183001) (width 0.25) (layer F.Cu) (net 6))
 (segment (start 119.709619 85.184999) (end 126.47262 91.948) (width 0.25) (layer F.Cu) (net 8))
 (segment (start 67.5386 83.8962) (end 118.44622 83.8962) (width 0.25) (layer F.Cu) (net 8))
 (segment (start 118.42082 83.8962) (end 119.709619 85.184999) (width 0.25) (layer F.Cu) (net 8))
 (segment (start 67.118599 83.476199) (end 67.5386 83.8962) (width 0.25) (layer F.Cu) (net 8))
 (segment (start 67.093199 83.476199) (end 67.118599 83.476199) (width 0.25) (layer F.Cu) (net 8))
 (segment (start 66.2432 82.6262) (end 67.093199 83.476199) (width 0.25) (layer F.Cu) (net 8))
 (segment (start 102.77442 82.6262) (end 108.69262 76.708) (width 0.25) (layer F.Cu) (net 7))
 (segment (start 68.7832 82.6262) (end 102.77442 82.6262) (width 0.25) (layer F.Cu) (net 7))
 (segment (start 173.736 77.893393) (end 175.674807 79.8322) (width 0.25) (layer F.Cu) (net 51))
 (segment (start 173.736 76.708) (end 173.736 77.893393) (width 0.25) (layer F.Cu) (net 51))
 (segment (start 196.047001 83.194201) (end 194.395401 83.194201) (width 0.25) (layer F.Cu) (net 51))
 (segment (start 196.747 83.8942) (end 196.047001 83.194201) (width 0.25) (layer F.Cu) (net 51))
 (segment (start 194.395401 83.194201) (end 191.0334 79.8322) (width 0.25) (layer F.Cu) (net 51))
 (segment (start 191.0334 79.8322) (end 175.674807 79.8322) (width 0.25) (layer F.Cu) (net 51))
 (segment (start 174.574199 83.489801) (end 174.650399 83.489801) (width 0.25) (layer F.Cu) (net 53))
 (segment (start 173.736 84.328) (end 174.574199 83.489801) (width 0.25) (layer F.Cu) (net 53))
 (segment (start 174.650399 83.489801) (end 176.276 81.8642) (width 0.25) (layer F.Cu) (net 53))
 (segment (start 176.276 81.8642) (end 190.6524 81.8642) (width 0.25) (layer F.Cu) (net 53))
 (segment (start 190.6524 81.8642) (end 190.6524 86.1822) (width 0.25) (layer F.Cu) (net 53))
 (segment (start 190.6524 86.1822) (end 192.4812 88.011) (width 0.25) (layer F.Cu) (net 53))
 (segment (start 199.287 84.9142) (end 198.0184 86.1828) (width 0.25) (layer F.Cu) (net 53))
 (segment (start 198.0184 86.1828) (end 198.0184 88.011) (width 0.25) (layer F.Cu) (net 53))
 (segment (start 198.0184 88.011) (end 192.4812 88.011) (width 0.25) (layer F.Cu) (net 53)))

